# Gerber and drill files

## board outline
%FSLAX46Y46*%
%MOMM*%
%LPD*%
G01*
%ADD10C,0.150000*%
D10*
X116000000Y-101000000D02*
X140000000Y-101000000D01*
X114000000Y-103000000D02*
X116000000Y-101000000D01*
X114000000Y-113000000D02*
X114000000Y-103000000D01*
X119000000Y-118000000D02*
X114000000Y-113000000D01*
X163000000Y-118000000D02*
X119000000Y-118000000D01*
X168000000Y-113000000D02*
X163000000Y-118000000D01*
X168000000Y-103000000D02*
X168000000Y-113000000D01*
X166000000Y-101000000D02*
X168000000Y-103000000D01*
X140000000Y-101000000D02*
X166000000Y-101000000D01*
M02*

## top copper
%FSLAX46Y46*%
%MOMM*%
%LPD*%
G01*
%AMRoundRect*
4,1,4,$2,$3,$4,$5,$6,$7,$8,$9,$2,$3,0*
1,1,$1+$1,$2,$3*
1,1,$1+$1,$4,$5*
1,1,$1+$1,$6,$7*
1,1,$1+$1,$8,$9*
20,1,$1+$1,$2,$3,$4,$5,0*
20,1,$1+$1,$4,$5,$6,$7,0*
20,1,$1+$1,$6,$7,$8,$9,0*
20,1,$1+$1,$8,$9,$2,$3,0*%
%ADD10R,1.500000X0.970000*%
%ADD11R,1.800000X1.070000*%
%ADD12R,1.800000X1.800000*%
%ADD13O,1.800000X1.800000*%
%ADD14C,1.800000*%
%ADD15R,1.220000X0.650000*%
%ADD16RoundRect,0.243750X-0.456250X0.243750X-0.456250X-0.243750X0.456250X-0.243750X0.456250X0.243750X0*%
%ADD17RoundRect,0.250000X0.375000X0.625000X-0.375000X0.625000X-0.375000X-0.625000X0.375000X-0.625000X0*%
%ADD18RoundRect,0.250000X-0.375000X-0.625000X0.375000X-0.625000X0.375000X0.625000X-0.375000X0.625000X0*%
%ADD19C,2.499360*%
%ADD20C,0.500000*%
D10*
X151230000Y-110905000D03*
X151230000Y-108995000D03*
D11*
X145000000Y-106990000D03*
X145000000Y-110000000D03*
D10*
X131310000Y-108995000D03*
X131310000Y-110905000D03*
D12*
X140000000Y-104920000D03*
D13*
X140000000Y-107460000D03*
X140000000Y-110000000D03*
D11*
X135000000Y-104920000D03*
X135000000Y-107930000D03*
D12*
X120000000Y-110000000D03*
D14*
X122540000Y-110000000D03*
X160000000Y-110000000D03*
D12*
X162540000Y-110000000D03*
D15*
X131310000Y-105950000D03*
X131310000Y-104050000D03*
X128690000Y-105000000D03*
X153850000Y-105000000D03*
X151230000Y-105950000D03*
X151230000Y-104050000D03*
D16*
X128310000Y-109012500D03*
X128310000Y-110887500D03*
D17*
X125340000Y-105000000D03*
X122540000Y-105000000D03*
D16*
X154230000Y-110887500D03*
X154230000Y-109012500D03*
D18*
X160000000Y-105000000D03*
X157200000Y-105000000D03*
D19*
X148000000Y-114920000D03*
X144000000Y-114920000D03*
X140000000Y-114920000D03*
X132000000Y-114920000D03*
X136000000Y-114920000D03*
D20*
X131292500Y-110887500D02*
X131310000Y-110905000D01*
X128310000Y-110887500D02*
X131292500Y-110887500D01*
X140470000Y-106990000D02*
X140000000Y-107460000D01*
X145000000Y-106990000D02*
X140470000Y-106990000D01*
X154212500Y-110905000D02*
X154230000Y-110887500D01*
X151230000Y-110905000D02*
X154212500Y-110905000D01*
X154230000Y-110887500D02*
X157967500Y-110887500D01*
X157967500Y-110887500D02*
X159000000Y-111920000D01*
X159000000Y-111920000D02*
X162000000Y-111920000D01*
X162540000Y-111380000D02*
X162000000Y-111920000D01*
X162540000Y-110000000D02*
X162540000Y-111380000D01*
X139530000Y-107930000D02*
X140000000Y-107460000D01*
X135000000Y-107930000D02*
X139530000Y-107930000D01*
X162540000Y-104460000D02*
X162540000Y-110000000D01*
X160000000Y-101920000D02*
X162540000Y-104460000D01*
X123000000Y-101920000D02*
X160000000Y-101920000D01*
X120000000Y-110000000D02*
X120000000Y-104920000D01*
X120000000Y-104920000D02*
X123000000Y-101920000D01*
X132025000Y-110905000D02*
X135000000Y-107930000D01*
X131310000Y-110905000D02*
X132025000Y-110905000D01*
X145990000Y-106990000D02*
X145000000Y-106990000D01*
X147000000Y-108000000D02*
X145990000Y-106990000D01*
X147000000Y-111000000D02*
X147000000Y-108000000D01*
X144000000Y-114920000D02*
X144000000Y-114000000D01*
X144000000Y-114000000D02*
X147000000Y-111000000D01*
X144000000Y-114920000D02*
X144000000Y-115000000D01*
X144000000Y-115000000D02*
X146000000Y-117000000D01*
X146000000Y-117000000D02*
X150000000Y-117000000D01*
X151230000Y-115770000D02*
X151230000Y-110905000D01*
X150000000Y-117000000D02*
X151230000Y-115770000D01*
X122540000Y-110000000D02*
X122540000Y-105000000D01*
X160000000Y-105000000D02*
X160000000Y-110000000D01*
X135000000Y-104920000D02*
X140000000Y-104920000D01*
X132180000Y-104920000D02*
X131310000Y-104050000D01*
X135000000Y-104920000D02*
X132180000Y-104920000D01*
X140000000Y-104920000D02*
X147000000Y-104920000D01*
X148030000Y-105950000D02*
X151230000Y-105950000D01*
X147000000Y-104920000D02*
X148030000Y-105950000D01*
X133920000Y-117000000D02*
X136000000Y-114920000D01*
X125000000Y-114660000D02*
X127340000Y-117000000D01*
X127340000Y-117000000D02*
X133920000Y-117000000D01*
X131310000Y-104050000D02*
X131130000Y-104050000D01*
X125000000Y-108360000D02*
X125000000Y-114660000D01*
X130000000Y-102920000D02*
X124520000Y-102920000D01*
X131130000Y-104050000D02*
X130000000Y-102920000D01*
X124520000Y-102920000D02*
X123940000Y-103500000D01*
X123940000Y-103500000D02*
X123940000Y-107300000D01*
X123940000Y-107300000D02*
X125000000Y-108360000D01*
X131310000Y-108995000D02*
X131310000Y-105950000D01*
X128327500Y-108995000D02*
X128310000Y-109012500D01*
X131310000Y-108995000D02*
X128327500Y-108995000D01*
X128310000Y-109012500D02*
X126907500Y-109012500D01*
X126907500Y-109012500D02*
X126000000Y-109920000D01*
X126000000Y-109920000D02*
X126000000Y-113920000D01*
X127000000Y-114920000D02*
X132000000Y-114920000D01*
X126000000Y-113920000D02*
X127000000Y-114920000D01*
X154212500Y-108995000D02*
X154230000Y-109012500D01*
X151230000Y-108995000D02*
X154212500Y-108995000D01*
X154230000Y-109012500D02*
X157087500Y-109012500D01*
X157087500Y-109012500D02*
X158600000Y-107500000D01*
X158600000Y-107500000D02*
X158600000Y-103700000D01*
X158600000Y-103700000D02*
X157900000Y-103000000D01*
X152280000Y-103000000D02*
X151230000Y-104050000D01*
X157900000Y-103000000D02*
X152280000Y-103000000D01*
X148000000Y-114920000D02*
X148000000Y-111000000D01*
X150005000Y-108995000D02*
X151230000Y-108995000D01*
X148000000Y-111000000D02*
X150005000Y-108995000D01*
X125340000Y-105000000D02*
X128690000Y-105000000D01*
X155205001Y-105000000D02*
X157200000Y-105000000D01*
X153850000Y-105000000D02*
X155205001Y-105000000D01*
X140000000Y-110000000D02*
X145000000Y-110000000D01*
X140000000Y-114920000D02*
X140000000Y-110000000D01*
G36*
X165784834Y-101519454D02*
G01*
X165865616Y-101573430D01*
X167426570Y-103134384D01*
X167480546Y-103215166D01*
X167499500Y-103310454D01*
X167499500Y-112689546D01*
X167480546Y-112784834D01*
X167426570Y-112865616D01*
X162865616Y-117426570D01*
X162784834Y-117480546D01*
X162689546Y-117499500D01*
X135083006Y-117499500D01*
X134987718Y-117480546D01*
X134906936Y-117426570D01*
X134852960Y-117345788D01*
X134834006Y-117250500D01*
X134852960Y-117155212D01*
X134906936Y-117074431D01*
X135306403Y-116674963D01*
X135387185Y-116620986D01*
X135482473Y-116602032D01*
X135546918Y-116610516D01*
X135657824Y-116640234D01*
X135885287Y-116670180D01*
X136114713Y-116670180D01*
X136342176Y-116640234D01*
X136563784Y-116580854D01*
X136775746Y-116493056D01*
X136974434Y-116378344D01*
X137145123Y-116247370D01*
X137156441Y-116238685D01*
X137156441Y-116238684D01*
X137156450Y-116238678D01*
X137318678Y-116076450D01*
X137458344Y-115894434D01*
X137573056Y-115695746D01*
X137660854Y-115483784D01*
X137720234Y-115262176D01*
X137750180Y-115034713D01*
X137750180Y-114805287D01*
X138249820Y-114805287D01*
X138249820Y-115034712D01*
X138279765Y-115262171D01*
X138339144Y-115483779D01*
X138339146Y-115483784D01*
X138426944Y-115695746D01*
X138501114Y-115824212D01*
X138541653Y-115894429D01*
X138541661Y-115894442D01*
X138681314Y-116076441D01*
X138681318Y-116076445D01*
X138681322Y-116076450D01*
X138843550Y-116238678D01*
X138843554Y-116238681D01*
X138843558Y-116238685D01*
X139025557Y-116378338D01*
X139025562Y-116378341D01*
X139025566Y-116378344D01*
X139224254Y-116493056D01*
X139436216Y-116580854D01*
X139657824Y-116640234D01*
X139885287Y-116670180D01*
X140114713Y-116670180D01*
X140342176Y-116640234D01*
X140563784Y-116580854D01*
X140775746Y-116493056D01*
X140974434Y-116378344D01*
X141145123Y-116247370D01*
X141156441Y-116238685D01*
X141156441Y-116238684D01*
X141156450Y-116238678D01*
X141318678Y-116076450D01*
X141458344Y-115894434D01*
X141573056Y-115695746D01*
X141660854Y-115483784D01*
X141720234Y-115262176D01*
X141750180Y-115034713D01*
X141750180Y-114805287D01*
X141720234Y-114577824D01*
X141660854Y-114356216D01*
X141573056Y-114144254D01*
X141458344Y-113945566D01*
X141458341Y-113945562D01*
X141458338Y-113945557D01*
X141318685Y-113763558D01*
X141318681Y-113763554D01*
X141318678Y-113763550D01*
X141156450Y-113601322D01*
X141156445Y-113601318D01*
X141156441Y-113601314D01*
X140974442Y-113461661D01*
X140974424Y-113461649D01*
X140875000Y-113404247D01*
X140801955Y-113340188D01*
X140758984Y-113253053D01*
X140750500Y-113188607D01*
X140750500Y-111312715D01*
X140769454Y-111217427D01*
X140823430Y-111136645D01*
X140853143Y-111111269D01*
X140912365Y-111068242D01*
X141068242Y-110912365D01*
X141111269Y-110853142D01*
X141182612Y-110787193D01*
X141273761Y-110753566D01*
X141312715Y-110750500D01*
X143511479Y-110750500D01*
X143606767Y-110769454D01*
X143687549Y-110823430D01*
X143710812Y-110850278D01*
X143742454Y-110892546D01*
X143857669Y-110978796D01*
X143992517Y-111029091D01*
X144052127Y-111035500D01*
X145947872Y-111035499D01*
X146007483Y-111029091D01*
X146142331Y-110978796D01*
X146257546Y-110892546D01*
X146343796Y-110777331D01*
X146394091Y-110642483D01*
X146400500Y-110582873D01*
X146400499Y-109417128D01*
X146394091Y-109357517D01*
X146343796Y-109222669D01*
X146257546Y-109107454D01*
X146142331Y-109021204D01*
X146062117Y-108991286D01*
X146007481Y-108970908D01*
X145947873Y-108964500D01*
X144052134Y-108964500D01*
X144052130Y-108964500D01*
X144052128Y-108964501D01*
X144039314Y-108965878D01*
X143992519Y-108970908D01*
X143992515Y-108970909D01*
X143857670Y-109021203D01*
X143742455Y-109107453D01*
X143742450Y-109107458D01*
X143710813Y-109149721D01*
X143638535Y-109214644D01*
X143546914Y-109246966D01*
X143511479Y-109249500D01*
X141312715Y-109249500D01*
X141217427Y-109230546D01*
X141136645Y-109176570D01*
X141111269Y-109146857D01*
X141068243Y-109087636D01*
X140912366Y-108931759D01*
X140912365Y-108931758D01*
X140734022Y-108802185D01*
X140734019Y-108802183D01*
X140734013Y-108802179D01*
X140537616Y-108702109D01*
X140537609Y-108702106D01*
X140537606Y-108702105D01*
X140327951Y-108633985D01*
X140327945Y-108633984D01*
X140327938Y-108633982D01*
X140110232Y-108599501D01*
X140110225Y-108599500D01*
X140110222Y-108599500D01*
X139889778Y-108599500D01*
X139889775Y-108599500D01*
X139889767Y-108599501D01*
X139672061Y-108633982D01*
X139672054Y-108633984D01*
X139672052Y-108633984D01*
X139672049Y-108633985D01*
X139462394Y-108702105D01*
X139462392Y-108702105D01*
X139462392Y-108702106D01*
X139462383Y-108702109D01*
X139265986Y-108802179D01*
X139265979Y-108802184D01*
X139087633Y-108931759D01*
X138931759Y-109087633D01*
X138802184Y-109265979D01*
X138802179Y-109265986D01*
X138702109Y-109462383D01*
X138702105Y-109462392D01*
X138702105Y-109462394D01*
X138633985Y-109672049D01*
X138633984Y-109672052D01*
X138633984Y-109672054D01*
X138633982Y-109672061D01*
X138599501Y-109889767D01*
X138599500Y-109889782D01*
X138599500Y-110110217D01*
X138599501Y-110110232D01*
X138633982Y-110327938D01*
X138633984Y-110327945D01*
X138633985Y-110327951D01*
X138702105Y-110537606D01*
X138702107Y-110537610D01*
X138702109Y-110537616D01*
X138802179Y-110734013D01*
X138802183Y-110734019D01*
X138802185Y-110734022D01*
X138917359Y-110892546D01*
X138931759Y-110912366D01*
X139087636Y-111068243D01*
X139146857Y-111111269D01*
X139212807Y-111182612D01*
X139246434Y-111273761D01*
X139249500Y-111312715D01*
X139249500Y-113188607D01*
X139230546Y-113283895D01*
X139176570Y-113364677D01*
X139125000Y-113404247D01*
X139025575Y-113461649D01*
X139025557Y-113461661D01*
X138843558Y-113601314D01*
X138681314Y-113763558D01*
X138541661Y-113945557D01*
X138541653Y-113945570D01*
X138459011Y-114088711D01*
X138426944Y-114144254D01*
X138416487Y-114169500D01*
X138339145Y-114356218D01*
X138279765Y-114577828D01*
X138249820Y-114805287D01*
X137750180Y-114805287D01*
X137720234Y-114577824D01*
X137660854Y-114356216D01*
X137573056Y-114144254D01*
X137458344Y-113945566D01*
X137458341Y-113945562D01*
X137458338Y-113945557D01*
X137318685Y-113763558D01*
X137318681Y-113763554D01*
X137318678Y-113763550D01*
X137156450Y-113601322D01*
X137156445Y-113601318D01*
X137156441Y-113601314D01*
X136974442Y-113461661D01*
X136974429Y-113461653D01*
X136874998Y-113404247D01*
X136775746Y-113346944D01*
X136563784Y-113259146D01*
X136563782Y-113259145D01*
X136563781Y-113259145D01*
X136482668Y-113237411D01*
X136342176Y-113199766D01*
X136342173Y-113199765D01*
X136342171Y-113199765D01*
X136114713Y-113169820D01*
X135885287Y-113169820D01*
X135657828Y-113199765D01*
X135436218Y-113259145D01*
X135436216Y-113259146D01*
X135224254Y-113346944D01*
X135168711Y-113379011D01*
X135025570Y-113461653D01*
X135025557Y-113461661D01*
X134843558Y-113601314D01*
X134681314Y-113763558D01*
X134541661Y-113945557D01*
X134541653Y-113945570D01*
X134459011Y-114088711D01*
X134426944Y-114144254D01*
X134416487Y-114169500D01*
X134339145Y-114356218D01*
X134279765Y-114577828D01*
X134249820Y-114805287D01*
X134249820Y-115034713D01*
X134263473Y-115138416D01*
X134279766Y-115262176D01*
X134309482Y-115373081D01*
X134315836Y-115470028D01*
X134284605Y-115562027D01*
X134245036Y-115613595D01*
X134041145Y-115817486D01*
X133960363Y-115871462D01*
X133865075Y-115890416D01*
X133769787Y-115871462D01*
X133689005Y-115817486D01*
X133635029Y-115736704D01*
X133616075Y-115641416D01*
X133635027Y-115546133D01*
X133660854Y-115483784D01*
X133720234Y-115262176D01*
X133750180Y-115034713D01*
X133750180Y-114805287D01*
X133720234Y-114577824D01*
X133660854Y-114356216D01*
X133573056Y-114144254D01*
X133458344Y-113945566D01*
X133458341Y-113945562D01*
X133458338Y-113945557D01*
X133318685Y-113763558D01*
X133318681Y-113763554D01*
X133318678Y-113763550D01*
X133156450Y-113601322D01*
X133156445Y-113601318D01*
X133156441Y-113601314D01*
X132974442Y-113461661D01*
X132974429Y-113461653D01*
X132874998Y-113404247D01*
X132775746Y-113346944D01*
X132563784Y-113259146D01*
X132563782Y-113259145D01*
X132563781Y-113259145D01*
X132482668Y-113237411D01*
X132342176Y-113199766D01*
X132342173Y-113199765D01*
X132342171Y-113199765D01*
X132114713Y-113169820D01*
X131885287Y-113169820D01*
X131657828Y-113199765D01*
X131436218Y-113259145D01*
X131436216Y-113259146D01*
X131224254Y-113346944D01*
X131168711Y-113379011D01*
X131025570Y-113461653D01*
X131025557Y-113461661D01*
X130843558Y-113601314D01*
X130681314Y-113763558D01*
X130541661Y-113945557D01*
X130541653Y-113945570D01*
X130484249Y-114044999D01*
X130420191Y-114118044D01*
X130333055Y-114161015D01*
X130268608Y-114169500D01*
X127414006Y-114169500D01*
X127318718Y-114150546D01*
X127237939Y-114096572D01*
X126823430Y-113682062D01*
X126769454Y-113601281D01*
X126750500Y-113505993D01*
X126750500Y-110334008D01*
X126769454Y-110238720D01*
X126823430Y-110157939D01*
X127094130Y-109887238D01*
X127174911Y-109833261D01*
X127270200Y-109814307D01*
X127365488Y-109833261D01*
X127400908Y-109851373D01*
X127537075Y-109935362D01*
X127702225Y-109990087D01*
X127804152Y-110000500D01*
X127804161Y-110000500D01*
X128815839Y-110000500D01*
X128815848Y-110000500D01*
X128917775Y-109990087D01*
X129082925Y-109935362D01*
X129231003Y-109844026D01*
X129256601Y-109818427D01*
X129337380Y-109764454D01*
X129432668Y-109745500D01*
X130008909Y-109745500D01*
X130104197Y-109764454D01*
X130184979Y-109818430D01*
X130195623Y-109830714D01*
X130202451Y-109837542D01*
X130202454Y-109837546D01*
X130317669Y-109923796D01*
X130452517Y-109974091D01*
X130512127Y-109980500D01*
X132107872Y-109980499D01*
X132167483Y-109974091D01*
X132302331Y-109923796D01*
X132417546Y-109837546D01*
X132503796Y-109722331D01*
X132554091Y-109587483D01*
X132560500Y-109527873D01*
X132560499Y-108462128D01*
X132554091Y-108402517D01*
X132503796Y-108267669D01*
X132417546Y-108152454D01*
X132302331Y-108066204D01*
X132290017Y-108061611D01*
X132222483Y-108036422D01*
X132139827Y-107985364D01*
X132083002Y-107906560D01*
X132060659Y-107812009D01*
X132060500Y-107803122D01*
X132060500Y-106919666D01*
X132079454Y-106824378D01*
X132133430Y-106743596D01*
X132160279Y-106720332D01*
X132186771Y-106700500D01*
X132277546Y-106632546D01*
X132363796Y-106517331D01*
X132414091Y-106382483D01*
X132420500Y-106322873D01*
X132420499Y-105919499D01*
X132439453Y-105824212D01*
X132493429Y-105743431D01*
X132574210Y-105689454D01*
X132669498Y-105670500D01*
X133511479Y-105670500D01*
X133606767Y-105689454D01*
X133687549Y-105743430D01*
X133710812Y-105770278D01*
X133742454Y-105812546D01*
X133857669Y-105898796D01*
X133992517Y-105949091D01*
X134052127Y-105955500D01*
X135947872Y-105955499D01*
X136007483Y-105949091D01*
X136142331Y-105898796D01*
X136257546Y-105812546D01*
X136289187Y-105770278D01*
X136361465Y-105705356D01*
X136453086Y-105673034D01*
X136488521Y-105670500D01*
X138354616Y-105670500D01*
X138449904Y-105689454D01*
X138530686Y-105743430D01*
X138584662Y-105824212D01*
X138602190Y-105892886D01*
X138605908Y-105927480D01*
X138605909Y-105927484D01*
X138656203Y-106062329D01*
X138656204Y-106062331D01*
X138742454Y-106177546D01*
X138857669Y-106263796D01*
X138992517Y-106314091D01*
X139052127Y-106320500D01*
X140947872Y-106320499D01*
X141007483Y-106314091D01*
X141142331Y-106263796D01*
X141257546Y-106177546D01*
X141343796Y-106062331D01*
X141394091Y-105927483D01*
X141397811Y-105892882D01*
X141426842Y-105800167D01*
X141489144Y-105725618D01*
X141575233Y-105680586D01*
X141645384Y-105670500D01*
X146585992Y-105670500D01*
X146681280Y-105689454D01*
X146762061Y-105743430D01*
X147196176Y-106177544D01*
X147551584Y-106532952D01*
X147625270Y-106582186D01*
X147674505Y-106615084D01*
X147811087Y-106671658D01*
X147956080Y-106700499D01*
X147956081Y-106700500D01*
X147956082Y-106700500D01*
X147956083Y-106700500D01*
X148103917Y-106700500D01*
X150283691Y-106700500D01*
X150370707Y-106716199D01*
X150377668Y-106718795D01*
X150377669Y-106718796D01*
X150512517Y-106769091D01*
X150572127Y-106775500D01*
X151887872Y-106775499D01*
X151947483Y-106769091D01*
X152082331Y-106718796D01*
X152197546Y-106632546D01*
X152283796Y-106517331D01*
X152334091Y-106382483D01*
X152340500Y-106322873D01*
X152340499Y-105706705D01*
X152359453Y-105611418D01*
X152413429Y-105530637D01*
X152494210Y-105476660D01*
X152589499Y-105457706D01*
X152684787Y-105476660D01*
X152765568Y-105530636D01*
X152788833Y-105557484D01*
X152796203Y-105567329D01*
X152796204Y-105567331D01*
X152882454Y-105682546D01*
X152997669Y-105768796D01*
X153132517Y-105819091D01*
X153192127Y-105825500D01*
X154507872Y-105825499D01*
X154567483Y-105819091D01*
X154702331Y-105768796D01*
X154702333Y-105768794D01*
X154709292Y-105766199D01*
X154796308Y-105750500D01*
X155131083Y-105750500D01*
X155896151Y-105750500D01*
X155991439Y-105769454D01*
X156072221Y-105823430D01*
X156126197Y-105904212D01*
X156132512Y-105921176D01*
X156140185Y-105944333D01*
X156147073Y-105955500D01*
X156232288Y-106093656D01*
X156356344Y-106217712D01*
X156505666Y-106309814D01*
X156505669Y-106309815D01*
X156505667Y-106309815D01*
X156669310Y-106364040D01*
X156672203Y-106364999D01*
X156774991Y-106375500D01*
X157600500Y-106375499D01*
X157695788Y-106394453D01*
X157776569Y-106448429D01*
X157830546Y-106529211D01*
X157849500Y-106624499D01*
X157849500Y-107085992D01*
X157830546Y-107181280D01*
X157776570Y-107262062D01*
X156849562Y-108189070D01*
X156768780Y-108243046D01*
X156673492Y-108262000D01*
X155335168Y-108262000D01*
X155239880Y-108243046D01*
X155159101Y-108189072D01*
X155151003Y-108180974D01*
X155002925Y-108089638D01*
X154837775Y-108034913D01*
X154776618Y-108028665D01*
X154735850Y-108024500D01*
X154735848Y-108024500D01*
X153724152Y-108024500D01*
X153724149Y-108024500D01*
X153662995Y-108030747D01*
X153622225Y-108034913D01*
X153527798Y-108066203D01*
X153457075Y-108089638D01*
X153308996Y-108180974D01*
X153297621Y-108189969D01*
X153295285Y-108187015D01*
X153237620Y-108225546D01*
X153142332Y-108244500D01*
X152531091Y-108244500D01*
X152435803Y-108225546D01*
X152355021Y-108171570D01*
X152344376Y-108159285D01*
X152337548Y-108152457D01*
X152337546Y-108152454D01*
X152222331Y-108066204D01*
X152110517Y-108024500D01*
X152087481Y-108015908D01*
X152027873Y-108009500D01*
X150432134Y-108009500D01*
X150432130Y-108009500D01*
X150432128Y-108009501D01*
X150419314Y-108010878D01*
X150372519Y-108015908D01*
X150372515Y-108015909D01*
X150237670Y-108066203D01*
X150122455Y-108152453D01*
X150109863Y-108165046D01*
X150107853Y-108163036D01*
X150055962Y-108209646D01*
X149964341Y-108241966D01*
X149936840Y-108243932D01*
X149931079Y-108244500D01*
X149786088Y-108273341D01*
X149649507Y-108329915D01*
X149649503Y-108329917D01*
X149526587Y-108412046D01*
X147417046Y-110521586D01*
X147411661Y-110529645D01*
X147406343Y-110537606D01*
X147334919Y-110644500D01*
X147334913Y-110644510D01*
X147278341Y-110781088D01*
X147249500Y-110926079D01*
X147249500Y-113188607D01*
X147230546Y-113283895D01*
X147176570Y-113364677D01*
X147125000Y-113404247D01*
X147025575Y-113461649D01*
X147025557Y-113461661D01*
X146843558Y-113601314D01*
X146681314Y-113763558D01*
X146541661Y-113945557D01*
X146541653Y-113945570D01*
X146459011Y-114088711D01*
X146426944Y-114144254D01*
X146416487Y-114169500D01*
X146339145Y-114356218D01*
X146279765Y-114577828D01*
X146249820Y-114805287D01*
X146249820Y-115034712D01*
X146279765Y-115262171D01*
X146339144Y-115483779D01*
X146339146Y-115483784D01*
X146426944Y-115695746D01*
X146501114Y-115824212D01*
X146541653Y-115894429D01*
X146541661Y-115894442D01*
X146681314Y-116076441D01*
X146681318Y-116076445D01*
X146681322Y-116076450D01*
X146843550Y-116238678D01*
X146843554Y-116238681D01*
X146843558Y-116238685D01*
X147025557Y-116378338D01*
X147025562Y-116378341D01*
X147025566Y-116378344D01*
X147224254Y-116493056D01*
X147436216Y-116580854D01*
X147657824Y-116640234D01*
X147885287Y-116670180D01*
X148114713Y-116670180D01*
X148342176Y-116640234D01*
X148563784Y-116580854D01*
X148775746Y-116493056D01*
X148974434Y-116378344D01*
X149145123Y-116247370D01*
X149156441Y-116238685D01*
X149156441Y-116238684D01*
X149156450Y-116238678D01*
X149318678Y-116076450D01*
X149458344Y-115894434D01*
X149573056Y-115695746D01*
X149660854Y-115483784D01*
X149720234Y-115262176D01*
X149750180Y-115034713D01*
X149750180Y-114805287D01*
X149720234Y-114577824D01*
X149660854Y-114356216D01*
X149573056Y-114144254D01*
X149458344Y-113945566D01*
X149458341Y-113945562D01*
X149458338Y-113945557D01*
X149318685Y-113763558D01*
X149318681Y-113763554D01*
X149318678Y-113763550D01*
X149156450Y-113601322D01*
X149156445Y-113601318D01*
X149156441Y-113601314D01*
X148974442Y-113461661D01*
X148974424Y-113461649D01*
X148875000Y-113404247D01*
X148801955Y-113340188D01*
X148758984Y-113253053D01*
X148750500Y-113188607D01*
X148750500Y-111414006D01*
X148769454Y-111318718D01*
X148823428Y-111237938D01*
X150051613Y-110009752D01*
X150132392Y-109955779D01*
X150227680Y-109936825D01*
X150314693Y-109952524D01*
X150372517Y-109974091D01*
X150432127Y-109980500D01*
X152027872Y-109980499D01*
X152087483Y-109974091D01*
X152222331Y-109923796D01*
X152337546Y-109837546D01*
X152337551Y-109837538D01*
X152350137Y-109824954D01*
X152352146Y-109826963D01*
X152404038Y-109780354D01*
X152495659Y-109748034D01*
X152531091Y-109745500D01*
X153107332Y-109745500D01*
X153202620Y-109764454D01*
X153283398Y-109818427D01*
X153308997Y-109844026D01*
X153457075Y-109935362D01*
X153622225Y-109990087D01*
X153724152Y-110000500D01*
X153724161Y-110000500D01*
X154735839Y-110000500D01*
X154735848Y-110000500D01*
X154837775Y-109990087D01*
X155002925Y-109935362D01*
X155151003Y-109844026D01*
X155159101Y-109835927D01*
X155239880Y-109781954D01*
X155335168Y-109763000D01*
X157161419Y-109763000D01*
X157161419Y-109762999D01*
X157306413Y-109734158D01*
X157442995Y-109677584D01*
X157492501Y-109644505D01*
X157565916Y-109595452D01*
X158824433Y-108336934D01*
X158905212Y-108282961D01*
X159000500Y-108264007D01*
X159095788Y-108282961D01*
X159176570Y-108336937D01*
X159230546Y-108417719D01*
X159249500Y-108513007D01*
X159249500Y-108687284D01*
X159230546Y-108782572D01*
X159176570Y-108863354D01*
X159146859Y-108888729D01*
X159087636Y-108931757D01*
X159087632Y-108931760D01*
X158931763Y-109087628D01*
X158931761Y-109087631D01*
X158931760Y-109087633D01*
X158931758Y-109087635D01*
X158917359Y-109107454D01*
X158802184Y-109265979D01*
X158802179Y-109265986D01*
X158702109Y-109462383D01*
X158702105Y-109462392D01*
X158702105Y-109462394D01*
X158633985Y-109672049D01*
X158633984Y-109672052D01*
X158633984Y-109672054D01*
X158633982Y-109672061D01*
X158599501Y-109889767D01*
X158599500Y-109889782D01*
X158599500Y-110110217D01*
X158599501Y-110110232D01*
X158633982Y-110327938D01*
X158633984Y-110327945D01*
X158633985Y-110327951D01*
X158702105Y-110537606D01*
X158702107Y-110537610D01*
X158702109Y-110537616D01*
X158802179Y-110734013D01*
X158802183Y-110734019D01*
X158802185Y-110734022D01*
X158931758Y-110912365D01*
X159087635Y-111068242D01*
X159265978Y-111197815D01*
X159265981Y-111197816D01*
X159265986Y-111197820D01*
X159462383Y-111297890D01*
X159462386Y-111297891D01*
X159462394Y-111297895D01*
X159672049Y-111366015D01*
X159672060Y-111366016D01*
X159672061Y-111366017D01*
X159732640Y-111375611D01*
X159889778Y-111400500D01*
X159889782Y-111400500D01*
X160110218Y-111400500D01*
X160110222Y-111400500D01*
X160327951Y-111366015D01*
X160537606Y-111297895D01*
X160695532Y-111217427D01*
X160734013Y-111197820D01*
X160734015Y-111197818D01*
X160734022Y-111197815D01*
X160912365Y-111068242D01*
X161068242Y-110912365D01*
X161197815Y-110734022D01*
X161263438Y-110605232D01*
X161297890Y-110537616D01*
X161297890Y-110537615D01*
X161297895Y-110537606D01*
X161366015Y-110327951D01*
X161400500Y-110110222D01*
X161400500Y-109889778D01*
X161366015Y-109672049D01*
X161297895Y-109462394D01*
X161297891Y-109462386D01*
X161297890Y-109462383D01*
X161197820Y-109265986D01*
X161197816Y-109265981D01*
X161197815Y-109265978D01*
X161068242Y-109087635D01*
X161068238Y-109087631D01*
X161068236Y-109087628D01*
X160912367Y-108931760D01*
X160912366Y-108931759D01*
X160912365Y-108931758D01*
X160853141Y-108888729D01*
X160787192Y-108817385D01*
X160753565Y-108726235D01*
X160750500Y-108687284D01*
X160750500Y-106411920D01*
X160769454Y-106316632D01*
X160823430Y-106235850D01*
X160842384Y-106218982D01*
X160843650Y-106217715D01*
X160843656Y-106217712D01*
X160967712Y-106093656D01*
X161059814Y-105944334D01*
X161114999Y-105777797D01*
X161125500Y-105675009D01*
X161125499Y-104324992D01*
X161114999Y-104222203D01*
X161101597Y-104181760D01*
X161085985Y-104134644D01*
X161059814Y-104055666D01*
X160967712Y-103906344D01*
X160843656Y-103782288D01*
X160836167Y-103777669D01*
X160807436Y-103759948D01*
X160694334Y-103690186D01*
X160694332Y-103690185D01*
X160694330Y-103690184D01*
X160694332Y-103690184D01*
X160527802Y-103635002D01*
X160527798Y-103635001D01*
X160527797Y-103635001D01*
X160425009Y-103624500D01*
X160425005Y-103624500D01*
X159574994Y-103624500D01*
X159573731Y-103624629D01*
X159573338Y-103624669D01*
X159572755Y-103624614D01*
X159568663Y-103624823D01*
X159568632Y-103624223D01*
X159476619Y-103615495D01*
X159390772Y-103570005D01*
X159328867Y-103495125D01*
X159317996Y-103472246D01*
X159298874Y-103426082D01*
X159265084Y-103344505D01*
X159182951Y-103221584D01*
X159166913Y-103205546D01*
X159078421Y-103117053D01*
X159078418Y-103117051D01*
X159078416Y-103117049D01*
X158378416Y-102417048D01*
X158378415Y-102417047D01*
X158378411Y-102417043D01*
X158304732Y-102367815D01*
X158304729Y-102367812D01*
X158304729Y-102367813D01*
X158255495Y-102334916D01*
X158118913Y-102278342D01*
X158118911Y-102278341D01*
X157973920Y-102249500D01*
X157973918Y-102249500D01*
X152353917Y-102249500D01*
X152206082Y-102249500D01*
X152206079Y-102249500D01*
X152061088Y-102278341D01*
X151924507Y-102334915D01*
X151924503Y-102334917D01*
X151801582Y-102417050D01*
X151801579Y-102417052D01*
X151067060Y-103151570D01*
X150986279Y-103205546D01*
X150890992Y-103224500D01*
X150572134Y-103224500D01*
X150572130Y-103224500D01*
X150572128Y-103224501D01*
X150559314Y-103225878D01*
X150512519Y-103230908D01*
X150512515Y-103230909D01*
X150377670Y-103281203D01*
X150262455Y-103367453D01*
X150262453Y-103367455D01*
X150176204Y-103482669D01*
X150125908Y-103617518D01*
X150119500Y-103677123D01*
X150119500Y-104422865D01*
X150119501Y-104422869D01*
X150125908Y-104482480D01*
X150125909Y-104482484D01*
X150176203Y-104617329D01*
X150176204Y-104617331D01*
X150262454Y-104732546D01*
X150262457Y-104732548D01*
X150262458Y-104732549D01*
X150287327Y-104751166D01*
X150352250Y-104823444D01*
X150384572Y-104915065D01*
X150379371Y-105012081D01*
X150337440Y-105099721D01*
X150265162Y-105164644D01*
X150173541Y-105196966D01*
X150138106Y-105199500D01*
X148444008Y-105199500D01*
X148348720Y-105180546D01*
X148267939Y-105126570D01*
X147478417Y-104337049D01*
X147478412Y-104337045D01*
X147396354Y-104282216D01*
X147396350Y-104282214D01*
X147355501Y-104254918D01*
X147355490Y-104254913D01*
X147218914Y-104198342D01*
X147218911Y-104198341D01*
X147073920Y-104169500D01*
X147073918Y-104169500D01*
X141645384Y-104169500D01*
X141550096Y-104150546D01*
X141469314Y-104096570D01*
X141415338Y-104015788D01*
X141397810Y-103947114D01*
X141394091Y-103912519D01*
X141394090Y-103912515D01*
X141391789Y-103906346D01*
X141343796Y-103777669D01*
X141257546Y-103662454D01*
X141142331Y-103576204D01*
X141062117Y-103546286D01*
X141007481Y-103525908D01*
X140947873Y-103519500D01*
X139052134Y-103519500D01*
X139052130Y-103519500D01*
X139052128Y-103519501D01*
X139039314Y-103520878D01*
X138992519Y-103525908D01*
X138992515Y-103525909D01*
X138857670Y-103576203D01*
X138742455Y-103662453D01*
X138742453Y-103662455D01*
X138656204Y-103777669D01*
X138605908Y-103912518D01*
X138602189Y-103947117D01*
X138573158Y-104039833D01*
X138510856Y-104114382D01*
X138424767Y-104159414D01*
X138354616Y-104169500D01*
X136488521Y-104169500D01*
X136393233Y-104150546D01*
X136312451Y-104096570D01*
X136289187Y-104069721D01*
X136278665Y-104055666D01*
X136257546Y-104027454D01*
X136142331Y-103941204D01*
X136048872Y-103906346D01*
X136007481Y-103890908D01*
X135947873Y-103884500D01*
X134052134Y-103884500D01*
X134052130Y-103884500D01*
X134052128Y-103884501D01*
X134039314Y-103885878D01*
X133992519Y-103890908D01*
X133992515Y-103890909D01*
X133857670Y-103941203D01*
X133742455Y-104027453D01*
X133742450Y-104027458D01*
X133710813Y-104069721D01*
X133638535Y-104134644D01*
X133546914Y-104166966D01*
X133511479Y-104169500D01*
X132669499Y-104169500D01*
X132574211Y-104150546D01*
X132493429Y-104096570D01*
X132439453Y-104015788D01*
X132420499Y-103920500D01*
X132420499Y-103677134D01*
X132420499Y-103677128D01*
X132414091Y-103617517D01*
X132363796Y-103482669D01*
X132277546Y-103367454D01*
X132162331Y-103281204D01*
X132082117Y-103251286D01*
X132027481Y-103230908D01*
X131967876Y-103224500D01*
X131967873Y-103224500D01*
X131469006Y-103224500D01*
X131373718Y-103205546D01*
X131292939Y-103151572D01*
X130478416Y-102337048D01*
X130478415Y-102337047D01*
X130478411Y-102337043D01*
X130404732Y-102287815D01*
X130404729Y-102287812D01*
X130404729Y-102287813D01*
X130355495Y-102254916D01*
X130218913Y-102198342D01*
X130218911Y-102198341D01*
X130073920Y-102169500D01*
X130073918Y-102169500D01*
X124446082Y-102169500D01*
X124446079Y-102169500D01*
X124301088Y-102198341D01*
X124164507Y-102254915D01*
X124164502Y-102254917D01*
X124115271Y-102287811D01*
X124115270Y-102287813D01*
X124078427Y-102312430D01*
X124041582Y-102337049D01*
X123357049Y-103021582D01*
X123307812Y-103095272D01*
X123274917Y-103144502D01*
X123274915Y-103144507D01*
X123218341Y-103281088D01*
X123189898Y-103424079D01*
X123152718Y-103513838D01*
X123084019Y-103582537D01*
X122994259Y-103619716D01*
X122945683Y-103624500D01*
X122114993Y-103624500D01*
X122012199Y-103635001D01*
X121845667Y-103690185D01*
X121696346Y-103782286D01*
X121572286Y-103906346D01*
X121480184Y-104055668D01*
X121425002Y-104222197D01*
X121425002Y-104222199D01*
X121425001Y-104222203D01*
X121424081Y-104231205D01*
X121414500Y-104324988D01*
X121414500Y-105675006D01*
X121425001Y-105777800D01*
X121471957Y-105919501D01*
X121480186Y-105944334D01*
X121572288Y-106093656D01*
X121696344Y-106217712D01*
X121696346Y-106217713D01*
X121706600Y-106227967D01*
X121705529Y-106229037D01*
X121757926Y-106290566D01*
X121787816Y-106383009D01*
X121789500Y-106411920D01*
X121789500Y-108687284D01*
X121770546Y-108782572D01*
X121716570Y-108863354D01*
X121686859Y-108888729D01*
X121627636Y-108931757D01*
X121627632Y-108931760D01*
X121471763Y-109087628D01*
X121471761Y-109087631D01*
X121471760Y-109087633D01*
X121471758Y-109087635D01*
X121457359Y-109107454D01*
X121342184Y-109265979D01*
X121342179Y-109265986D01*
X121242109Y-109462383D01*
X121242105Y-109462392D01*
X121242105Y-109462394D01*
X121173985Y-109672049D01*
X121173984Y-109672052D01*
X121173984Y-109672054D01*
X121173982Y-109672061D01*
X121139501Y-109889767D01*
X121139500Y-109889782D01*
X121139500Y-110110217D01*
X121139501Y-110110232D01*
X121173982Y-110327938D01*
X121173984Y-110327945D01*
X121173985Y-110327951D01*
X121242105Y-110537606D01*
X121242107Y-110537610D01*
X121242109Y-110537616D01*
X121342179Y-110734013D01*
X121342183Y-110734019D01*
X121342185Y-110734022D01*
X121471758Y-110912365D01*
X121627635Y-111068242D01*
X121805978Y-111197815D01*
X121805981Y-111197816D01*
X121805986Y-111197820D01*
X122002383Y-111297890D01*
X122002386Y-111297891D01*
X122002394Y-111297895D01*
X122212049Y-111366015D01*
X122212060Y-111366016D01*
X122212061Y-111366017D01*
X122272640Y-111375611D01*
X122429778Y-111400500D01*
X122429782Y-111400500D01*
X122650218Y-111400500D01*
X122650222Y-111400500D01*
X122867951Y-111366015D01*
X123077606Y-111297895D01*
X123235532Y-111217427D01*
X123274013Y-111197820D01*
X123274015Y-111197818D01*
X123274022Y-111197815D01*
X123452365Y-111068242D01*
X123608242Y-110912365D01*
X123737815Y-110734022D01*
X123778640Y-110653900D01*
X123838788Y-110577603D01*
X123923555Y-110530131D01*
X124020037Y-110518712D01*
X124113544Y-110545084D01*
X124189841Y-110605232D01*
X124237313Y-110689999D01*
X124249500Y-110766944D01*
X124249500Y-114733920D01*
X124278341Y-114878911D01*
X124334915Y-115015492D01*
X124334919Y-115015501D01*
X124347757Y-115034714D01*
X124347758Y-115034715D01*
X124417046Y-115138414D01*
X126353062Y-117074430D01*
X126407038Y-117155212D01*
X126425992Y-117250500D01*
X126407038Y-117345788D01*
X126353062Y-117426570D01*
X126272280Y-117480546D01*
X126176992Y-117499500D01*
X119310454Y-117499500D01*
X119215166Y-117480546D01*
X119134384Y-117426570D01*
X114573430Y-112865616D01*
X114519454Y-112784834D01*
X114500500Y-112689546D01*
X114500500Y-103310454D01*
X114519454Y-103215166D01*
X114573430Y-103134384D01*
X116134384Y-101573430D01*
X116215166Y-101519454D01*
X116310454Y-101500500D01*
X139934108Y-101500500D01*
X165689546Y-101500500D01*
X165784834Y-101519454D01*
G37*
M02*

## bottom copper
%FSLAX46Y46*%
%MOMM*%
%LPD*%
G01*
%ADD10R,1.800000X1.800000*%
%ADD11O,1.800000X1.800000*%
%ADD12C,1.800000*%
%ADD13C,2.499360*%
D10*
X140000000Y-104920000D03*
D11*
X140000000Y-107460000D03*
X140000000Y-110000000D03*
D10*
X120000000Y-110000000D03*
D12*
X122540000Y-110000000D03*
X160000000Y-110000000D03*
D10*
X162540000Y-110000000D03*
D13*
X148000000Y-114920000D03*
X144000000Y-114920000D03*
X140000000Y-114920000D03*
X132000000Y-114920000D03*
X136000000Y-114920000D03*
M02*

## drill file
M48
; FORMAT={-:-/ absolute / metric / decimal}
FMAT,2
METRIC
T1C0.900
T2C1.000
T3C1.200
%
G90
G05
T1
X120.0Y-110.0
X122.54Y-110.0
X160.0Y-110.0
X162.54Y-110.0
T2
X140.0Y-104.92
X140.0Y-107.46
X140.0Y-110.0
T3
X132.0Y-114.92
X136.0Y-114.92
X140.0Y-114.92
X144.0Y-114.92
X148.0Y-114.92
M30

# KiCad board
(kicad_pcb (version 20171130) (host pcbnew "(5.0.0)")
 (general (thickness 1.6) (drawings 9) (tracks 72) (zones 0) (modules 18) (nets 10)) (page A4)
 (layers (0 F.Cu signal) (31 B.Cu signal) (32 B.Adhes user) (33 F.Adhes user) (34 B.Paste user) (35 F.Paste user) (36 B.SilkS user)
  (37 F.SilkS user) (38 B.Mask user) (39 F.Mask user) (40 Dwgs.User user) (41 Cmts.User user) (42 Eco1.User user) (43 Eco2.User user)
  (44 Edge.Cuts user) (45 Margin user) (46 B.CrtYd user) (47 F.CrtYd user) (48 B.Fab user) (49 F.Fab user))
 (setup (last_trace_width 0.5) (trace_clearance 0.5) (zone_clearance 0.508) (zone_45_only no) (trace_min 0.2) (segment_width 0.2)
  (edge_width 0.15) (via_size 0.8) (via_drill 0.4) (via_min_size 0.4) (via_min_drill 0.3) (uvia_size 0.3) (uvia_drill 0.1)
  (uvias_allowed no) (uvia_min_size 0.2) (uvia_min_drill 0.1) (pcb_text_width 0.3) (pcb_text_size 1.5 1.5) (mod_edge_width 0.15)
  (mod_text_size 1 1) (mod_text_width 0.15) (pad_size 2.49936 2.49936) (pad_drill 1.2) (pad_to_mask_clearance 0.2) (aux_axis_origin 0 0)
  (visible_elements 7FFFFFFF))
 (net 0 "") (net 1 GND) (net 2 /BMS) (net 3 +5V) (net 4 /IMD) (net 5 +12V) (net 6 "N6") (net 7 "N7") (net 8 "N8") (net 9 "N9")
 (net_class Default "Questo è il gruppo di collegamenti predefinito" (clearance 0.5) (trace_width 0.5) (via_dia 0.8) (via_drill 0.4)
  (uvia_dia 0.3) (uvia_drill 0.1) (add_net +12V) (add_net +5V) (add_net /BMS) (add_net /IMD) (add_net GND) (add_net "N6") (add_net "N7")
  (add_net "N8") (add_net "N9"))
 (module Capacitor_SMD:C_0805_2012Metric (layer F.Cu) (at 151.23 109.95 270)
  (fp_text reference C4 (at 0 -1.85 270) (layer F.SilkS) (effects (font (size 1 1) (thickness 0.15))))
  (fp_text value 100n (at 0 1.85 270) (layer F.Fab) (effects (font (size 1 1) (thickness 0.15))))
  (pad 2 smd rect (at 0.955 0 270) (size 0.97 1.5) (layers F.Cu F.Paste F.Mask) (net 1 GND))
  (pad 1 smd rect (at -0.955 0 270) (size 0.97 1.5) (layers F.Cu F.Paste F.Mask) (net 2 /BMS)))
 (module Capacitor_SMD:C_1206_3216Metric (layer F.Cu) (at 145 108.495 90)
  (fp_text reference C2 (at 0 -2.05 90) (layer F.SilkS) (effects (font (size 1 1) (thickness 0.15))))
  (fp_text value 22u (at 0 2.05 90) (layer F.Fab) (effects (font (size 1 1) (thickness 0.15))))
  (pad 2 smd rect (at 1.505 0 90) (size 1.07 1.8) (layers F.Cu F.Paste F.Mask) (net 1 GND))
  (pad 1 smd rect (at -1.505 0 90) (size 1.07 1.8) (layers F.Cu F.Paste F.Mask) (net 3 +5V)))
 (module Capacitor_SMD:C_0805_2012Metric (layer F.Cu) (at 131.31 109.95 270)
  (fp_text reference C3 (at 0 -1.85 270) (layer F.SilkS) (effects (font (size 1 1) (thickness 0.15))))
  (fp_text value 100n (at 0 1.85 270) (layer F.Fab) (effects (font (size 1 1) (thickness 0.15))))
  (pad 1 smd rect (at -0.955 0 270) (size 0.97 1.5) (layers F.Cu F.Paste F.Mask) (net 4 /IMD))
  (pad 2 smd rect (at 0.955 0 270) (size 0.97 1.5) (layers F.Cu F.Paste F.Mask) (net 1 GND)))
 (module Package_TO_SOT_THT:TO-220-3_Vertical (layer F.Cu) (at 140 104.92 270)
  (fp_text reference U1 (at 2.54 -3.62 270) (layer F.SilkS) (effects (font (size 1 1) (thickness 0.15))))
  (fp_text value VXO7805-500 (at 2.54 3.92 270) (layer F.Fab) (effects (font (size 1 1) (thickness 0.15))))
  (pad 1 thru_hole rect (at 0 0 270) (size 1.8 1.8) (drill 1) (layers *.Cu *.Mask) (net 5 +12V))
  (pad 2 thru_hole oval (at 2.54 0 270) (size 1.8 1.8) (drill 1) (layers *.Cu *.Mask) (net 1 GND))
  (pad 3 thru_hole oval (at 5.08 0 270) (size 1.8 1.8) (drill 1) (layers *.Cu *.Mask) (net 3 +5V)))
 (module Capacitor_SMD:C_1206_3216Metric (layer F.Cu) (at 135 106.425 270)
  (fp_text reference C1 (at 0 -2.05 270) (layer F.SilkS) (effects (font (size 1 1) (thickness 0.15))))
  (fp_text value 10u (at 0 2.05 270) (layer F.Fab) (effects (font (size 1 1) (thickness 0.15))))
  (pad 1 smd rect (at -1.505 0 270) (size 1.07 1.8) (layers F.Cu F.Paste F.Mask) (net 5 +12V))
  (pad 2 smd rect (at 1.505 0 270) (size 1.07 1.8) (layers F.Cu F.Paste F.Mask) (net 1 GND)))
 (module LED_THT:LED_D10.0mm (layer B.Cu) (at 120 110)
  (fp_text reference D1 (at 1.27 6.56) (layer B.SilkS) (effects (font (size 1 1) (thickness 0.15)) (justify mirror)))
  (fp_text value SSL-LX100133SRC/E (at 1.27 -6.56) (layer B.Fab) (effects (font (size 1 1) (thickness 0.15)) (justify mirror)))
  (pad 1 thru_hole rect (at 0 0) (size 1.8 1.8) (drill 0.9) (layers *.Cu *.Mask) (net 1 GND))
  (pad 2 thru_hole circle (at 2.54 0) (size 1.8 1.8) (drill 0.9) (layers *.Cu *.Mask) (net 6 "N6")))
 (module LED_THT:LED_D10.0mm (layer B.Cu) (at 162.54 110 180)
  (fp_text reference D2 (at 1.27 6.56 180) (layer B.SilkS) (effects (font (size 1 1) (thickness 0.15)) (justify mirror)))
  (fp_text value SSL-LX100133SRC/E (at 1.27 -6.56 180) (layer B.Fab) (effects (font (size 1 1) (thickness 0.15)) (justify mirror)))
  (pad 2 thru_hole circle (at 2.54 0 180) (size 1.8 1.8) (drill 0.9) (layers *.Cu *.Mask) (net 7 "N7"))
  (pad 1 thru_hole rect (at 0 0 180) (size 1.8 1.8) (drill 0.9) (layers *.Cu *.Mask) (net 1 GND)))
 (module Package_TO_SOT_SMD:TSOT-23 (layer F.Cu) (at 130 105 180)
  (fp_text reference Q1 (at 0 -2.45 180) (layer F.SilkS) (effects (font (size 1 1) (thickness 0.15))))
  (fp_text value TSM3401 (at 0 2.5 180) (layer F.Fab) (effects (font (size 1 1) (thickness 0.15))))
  (pad 1 smd rect (at -1.31 -0.95 180) (size 1.22 0.65) (layers F.Cu F.Paste F.Mask) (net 4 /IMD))
  (pad 2 smd rect (at -1.31 0.95 180) (size 1.22 0.65) (layers F.Cu F.Paste F.Mask) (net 5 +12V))
  (pad 3 smd rect (at 1.31 0 180) (size 1.22 0.65) (layers F.Cu F.Paste F.Mask) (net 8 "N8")))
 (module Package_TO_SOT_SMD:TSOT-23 (layer F.Cu) (at 152.54 105)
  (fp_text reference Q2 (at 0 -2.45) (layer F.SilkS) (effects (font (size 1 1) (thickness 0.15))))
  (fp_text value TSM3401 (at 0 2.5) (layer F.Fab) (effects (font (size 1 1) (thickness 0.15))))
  (pad 3 smd rect (at 1.31 0) (size 1.22 0.65) (layers F.Cu F.Paste F.Mask) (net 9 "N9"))
  (pad 2 smd rect (at -1.31 0.95) (size 1.22 0.65) (layers F.Cu F.Paste F.Mask) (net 5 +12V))
  (pad 1 smd rect (at -1.31 -0.95) (size 1.22 0.65) (layers F.Cu F.Paste F.Mask) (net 2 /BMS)))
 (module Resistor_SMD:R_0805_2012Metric (layer F.Cu) (at 128.31 109.95 270)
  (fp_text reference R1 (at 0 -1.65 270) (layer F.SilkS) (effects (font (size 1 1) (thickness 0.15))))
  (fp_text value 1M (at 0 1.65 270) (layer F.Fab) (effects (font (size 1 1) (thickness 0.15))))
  (pad 1 smd roundrect (at -0.9375 0 270) (size 0.975 1.4) (layers F.Cu F.Paste F.Mask) (roundrect_rratio 0.25) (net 4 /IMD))
  (pad 2 smd roundrect (at 0.9375 0 270) (size 0.975 1.4) (layers F.Cu F.Paste F.Mask) (roundrect_rratio 0.25) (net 1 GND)))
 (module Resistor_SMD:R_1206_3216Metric (layer F.Cu) (at 123.94 105 180)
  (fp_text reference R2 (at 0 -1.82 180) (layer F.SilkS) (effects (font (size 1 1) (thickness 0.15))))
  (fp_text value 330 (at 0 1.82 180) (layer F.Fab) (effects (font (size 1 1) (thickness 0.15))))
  (pad 1 smd roundrect (at -1.4 0 180) (size 1.25 1.75) (layers F.Cu F.Paste F.Mask) (roundrect_rratio 0.2) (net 8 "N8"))
  (pad 2 smd roundrect (at 1.4 0 180) (size 1.25 1.75) (layers F.Cu F.Paste F.Mask) (roundrect_rratio 0.2) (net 6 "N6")))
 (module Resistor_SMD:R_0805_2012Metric (layer F.Cu) (at 154.23 109.95 270)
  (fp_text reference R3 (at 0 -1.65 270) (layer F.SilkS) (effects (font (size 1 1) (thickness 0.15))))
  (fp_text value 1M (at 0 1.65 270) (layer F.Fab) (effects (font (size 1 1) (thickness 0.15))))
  (pad 2 smd roundrect (at 0.9375 0 270) (size 0.975 1.4) (layers F.Cu F.Paste F.Mask) (roundrect_rratio 0.25) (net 1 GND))
  (pad 1 smd roundrect (at -0.9375 0 270) (size 0.975 1.4) (layers F.Cu F.Paste F.Mask) (roundrect_rratio 0.25) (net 2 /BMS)))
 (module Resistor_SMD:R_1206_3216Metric (layer F.Cu) (at 158.6 105)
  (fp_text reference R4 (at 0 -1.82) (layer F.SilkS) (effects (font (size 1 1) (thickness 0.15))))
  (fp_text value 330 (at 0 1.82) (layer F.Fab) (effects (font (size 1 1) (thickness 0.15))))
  (pad 2 smd roundrect (at 1.4 0) (size 1.25 1.75) (layers F.Cu F.Paste F.Mask) (roundrect_rratio 0.2) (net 7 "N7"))
  (pad 1 smd roundrect (at -1.4 0) (size 1.25 1.75) (layers F.Cu F.Paste F.Mask) (roundrect_rratio 0.2) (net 9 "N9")))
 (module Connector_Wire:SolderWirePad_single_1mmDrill (layer F.Cu) (at 148 114.92)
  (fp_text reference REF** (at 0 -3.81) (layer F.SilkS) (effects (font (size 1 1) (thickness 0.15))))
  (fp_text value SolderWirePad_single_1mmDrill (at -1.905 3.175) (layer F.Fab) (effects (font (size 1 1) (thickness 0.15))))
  (pad 1 thru_hole circle (at 0 0) (size 2.49936 2.49936) (drill 1.2) (layers *.Cu *.Mask) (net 2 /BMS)))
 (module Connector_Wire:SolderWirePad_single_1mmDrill (layer F.Cu) (at 144 114.92)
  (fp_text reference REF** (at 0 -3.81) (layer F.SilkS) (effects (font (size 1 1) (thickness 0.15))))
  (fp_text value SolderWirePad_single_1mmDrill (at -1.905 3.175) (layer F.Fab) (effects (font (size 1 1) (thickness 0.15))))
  (pad 1 thru_hole circle (at 0 0) (size 2.49936 2.49936) (drill 1.2) (layers *.Cu *.Mask) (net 1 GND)))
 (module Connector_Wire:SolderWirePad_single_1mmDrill (layer F.Cu) (at 140 114.92)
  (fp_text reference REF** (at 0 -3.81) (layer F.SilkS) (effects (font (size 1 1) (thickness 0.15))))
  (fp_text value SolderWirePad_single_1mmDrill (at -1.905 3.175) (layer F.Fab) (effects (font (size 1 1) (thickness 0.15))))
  (pad 1 thru_hole circle (at 0 0) (size 2.49936 2.49936) (drill 1.2) (layers *.Cu *.Mask) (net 3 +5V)))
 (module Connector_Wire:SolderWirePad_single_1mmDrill (layer F.Cu) (at 132 114.92)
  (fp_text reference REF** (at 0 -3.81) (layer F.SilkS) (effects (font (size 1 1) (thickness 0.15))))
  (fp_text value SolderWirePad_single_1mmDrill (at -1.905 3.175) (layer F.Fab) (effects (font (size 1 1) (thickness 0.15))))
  (pad 1 thru_hole circle (at 0 0) (size 2.49936 2.49936) (drill 1.2) (layers *.Cu *.Mask) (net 4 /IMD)))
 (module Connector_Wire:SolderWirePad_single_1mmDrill (layer F.Cu) (at 136 114.92)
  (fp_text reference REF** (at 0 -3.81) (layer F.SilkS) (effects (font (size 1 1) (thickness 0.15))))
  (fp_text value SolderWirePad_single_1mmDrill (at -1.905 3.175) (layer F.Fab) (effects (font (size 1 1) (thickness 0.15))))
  (pad 1 thru_hole circle (at 0 0) (size 2.49936 2.49936) (drill 1.2) (layers *.Cu *.Mask) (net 5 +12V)))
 (gr_line (start 116 101) (end 140 101) (layer Edge.Cuts) (width 0.15))
 (gr_line (start 114 103) (end 116 101) (layer Edge.Cuts) (width 0.15))
 (gr_line (start 114 113) (end 114 103) (layer Edge.Cuts) (width 0.15))
 (gr_line (start 119 118) (end 114 113) (layer Edge.Cuts) (width 0.15))
 (gr_line (start 163 118) (end 119 118) (layer Edge.Cuts) (width 0.15))
 (gr_line (start 168 113) (end 163 118) (layer Edge.Cuts) (width 0.15))
 (gr_line (start 168 103) (end 168 113) (layer Edge.Cuts) (width 0.15))
 (gr_line (start 166 101) (end 168 103) (layer Edge.Cuts) (width 0.15))
 (gr_line (start 140 101) (end 166 101) (layer Edge.Cuts) (width 0.15))
 (segment (start 131.2925 110.8875) (end 131.31 110.905) (width 0.5) (layer F.Cu) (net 1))
 (segment (start 128.31 110.8875) (end 131.2925 110.8875) (width 0.5) (layer F.Cu) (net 1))
 (segment (start 140.47 106.99) (end 140 107.46) (width 0.5) (layer F.Cu) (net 1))
 (segment (start 145 106.99) (end 140.47 106.99) (width 0.5) (layer F.Cu) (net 1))
 (segment (start 154.2125 110.905) (end 154.23 110.8875) (width 0.5) (layer F.Cu) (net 1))
 (segment (start 151.23 110.905) (end 154.2125 110.905) (width 0.5) (layer F.Cu) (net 1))
 (segment (start 154.23 110.8875) (end 157.9675 110.8875) (width 0.5) (layer F.Cu) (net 1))
 (segment (start 157.9675 110.8875) (end 159 111.92) (width 0.5) (layer F.Cu) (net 1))
 (segment (start 159 111.92) (end 162 111.92) (width 0.5) (layer F.Cu) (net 1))
 (segment (start 162.54 111.38) (end 162 111.92) (width 0.5) (layer F.Cu) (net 1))
 (segment (start 162.54 110) (end 162.54 111.38) (width 0.5) (layer F.Cu) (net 1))
 (segment (start 139.53 107.93) (end 140 107.46) (width 0.5) (layer F.Cu) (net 1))
 (segment (start 135 107.93) (end 139.53 107.93) (width 0.5) (layer F.Cu) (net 1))
 (segment (start 162.54 104.46) (end 162.54 110) (width 0.5) (layer F.Cu) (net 1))
 (segment (start 160 101.92) (end 162.54 104.46) (width 0.5) (layer F.Cu) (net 1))
 (segment (start 123 101.92) (end 160 101.92) (width 0.5) (layer F.Cu) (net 1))
 (segment (start 120 110) (end 120 104.92) (width 0.5) (layer F.Cu) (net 1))
 (segment (start 120 104.92) (end 123 101.92) (width 0.5) (layer F.Cu) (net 1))
 (segment (start 132.025 110.905) (end 135 107.93) (width 0.5) (layer F.Cu) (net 1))
 (segment (start 131.31 110.905) (end 132.025 110.905) (width 0.5) (layer F.Cu) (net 1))
 (segment (start 145.99 106.99) (end 145 106.99) (width 0.5) (layer F.Cu) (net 1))
 (segment (start 147 108) (end 145.99 106.99) (width 0.5) (layer F.Cu) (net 1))
 (segment (start 147 111) (end 147 108) (width 0.5) (layer F.Cu) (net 1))
 (segment (start 144 114.92) (end 144 114) (width 0.5) (layer F.Cu) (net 1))
 (segment (start 144 114) (end 147 111) (width 0.5) (layer F.Cu) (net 1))
 (segment (start 144 114.92) (end 144 115) (width 0.5) (layer F.Cu) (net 1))
 (segment (start 144 115) (end 146 117) (width 0.5) (layer F.Cu) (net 1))
 (segment (start 146 117) (end 150 117) (width 0.5) (layer F.Cu) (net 1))
 (segment (start 151.23 115.77) (end 151.23 110.905) (width 0.5) (layer F.Cu) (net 1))
 (segment (start 150 117) (end 151.23 115.77) (width 0.5) (layer F.Cu) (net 1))
 (segment (start 122.54 110) (end 122.54 105) (width 0.5) (layer F.Cu) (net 6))
 (segment (start 160 105) (end 160 110) (width 0.5) (layer F.Cu) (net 7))
 (segment (start 135 104.92) (end 140 104.92) (width 0.5) (layer F.Cu) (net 5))
 (segment (start 132.18 104.92) (end 131.31 104.05) (width 0.5) (layer F.Cu) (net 5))
 (segment (start 135 104.92) (end 132.18 104.92) (width 0.5) (layer F.Cu) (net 5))
 (segment (start 140 104.92) (end 147 104.92) (width 0.5) (layer F.Cu) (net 5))
 (segment (start 148.03 105.95) (end 151.23 105.95) (width 0.5) (layer F.Cu) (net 5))
 (segment (start 147 104.92) (end 148.03 105.95) (width 0.5) (layer F.Cu) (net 5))
 (segment (start 133.92 117) (end 136 114.92) (width 0.5) (layer F.Cu) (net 5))
 (segment (start 125 114.66) (end 127.34 117) (width 0.5) (layer F.Cu) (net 5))
 (segment (start 127.34 117) (end 133.92 117) (width 0.5) (layer F.Cu) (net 5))
 (segment (start 131.31 104.05) (end 131.13 104.05) (width 0.5) (layer F.Cu) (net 5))
 (segment (start 125 108.36) (end 125 114.66) (width 0.5) (layer F.Cu) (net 5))
 (segment (start 130 102.92) (end 124.52 102.92) (width 0.5) (layer F.Cu) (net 5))
 (segment (start 131.13 104.05) (end 130 102.92) (width 0.5) (layer F.Cu) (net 5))
 (segment (start 124.52 102.92) (end 123.94 103.5) (width 0.5) (layer F.Cu) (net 5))
 (segment (start 123.94 103.5) (end 123.94 107.3) (width 0.5) (layer F.Cu) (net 5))
 (segment (start 123.94 107.3) (end 125 108.36) (width 0.5) (layer F.Cu) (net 5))
 (segment (start 131.31 108.995) (end 131.31 105.95) (width 0.5) (layer F.Cu) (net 4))
 (segment (start 128.3275 108.995) (end 128.31 109.0125) (width 0.5) (layer F.Cu) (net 4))
 (segment (start 131.31 108.995) (end 128.3275 108.995) (width 0.5) (layer F.Cu) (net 4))
 (segment (start 128.31 109.0125) (end 126.9075 109.0125) (width 0.5) (layer F.Cu) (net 4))
 (segment (start 126.9075 109.0125) (end 126 109.92) (width 0.5) (layer F.Cu) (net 4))
 (segment (start 126 109.92) (end 126 113.92) (width 0.5) (layer F.Cu) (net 4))
 (segment (start 127 114.92) (end 132 114.92) (width 0.5) (layer F.Cu) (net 4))
 (segment (start 126 113.92) (end 127 114.92) (width 0.5) (layer F.Cu) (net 4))
 (segment (start 154.2125 108.995) (end 154.23 109.0125) (width 0.5) (layer F.Cu) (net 2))
 (segment (start 151.23 108.995) (end 154.2125 108.995) (width 0.5) (layer F.Cu) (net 2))
 (segment (start 154.23 109.0125) (end 157.0875 109.0125) (width 0.5) (layer F.Cu) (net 2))
 (segment (start 157.0875 109.0125) (end 158.6 107.5) (width 0.5) (layer F.Cu) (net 2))
 (segment (start 158.6 107.5) (end 158.6 103.7) (width 0.5) (layer F.Cu) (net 2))
 (segment (start 158.6 103.7) (end 157.9 103) (width 0.5) (layer F.Cu) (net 2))
 (segment (start 152.28 103) (end 151.23 104.05) (width 0.5) (layer F.Cu) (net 2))
 (segment (start 157.9 103) (end 152.28 103) (width 0.5) (layer F.Cu) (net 2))
 (segment (start 148 114.92) (end 148 111) (width 0.5) (layer F.Cu) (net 2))
 (segment (start 150.005 108.995) (end 151.23 108.995) (width 0.5) (layer F.Cu) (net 2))
 (segment (start 148 111) (end 150.005 108.995) (width 0.5) (layer F.Cu) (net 2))
 (segment (start 125.34 105) (end 128.69 105) (width 0.5) (layer F.Cu) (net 8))
 (segment (start 155.205001 105) (end 157.2 105) (width 0.5) (layer F.Cu) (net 9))
 (segment (start 153.85 105) (end 155.205001 105) (width 0.5) (layer F.Cu) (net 9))
 (segment (start 140 110) (end 145 110) (width 0.5) (layer F.Cu) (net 3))
 (segment (start 140 114.92) (end 140 110) (width 0.5) (layer F.Cu) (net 3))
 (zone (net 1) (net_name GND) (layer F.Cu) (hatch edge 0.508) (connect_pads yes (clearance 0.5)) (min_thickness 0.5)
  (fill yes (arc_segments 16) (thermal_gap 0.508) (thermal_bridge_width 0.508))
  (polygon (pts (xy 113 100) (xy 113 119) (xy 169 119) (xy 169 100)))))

